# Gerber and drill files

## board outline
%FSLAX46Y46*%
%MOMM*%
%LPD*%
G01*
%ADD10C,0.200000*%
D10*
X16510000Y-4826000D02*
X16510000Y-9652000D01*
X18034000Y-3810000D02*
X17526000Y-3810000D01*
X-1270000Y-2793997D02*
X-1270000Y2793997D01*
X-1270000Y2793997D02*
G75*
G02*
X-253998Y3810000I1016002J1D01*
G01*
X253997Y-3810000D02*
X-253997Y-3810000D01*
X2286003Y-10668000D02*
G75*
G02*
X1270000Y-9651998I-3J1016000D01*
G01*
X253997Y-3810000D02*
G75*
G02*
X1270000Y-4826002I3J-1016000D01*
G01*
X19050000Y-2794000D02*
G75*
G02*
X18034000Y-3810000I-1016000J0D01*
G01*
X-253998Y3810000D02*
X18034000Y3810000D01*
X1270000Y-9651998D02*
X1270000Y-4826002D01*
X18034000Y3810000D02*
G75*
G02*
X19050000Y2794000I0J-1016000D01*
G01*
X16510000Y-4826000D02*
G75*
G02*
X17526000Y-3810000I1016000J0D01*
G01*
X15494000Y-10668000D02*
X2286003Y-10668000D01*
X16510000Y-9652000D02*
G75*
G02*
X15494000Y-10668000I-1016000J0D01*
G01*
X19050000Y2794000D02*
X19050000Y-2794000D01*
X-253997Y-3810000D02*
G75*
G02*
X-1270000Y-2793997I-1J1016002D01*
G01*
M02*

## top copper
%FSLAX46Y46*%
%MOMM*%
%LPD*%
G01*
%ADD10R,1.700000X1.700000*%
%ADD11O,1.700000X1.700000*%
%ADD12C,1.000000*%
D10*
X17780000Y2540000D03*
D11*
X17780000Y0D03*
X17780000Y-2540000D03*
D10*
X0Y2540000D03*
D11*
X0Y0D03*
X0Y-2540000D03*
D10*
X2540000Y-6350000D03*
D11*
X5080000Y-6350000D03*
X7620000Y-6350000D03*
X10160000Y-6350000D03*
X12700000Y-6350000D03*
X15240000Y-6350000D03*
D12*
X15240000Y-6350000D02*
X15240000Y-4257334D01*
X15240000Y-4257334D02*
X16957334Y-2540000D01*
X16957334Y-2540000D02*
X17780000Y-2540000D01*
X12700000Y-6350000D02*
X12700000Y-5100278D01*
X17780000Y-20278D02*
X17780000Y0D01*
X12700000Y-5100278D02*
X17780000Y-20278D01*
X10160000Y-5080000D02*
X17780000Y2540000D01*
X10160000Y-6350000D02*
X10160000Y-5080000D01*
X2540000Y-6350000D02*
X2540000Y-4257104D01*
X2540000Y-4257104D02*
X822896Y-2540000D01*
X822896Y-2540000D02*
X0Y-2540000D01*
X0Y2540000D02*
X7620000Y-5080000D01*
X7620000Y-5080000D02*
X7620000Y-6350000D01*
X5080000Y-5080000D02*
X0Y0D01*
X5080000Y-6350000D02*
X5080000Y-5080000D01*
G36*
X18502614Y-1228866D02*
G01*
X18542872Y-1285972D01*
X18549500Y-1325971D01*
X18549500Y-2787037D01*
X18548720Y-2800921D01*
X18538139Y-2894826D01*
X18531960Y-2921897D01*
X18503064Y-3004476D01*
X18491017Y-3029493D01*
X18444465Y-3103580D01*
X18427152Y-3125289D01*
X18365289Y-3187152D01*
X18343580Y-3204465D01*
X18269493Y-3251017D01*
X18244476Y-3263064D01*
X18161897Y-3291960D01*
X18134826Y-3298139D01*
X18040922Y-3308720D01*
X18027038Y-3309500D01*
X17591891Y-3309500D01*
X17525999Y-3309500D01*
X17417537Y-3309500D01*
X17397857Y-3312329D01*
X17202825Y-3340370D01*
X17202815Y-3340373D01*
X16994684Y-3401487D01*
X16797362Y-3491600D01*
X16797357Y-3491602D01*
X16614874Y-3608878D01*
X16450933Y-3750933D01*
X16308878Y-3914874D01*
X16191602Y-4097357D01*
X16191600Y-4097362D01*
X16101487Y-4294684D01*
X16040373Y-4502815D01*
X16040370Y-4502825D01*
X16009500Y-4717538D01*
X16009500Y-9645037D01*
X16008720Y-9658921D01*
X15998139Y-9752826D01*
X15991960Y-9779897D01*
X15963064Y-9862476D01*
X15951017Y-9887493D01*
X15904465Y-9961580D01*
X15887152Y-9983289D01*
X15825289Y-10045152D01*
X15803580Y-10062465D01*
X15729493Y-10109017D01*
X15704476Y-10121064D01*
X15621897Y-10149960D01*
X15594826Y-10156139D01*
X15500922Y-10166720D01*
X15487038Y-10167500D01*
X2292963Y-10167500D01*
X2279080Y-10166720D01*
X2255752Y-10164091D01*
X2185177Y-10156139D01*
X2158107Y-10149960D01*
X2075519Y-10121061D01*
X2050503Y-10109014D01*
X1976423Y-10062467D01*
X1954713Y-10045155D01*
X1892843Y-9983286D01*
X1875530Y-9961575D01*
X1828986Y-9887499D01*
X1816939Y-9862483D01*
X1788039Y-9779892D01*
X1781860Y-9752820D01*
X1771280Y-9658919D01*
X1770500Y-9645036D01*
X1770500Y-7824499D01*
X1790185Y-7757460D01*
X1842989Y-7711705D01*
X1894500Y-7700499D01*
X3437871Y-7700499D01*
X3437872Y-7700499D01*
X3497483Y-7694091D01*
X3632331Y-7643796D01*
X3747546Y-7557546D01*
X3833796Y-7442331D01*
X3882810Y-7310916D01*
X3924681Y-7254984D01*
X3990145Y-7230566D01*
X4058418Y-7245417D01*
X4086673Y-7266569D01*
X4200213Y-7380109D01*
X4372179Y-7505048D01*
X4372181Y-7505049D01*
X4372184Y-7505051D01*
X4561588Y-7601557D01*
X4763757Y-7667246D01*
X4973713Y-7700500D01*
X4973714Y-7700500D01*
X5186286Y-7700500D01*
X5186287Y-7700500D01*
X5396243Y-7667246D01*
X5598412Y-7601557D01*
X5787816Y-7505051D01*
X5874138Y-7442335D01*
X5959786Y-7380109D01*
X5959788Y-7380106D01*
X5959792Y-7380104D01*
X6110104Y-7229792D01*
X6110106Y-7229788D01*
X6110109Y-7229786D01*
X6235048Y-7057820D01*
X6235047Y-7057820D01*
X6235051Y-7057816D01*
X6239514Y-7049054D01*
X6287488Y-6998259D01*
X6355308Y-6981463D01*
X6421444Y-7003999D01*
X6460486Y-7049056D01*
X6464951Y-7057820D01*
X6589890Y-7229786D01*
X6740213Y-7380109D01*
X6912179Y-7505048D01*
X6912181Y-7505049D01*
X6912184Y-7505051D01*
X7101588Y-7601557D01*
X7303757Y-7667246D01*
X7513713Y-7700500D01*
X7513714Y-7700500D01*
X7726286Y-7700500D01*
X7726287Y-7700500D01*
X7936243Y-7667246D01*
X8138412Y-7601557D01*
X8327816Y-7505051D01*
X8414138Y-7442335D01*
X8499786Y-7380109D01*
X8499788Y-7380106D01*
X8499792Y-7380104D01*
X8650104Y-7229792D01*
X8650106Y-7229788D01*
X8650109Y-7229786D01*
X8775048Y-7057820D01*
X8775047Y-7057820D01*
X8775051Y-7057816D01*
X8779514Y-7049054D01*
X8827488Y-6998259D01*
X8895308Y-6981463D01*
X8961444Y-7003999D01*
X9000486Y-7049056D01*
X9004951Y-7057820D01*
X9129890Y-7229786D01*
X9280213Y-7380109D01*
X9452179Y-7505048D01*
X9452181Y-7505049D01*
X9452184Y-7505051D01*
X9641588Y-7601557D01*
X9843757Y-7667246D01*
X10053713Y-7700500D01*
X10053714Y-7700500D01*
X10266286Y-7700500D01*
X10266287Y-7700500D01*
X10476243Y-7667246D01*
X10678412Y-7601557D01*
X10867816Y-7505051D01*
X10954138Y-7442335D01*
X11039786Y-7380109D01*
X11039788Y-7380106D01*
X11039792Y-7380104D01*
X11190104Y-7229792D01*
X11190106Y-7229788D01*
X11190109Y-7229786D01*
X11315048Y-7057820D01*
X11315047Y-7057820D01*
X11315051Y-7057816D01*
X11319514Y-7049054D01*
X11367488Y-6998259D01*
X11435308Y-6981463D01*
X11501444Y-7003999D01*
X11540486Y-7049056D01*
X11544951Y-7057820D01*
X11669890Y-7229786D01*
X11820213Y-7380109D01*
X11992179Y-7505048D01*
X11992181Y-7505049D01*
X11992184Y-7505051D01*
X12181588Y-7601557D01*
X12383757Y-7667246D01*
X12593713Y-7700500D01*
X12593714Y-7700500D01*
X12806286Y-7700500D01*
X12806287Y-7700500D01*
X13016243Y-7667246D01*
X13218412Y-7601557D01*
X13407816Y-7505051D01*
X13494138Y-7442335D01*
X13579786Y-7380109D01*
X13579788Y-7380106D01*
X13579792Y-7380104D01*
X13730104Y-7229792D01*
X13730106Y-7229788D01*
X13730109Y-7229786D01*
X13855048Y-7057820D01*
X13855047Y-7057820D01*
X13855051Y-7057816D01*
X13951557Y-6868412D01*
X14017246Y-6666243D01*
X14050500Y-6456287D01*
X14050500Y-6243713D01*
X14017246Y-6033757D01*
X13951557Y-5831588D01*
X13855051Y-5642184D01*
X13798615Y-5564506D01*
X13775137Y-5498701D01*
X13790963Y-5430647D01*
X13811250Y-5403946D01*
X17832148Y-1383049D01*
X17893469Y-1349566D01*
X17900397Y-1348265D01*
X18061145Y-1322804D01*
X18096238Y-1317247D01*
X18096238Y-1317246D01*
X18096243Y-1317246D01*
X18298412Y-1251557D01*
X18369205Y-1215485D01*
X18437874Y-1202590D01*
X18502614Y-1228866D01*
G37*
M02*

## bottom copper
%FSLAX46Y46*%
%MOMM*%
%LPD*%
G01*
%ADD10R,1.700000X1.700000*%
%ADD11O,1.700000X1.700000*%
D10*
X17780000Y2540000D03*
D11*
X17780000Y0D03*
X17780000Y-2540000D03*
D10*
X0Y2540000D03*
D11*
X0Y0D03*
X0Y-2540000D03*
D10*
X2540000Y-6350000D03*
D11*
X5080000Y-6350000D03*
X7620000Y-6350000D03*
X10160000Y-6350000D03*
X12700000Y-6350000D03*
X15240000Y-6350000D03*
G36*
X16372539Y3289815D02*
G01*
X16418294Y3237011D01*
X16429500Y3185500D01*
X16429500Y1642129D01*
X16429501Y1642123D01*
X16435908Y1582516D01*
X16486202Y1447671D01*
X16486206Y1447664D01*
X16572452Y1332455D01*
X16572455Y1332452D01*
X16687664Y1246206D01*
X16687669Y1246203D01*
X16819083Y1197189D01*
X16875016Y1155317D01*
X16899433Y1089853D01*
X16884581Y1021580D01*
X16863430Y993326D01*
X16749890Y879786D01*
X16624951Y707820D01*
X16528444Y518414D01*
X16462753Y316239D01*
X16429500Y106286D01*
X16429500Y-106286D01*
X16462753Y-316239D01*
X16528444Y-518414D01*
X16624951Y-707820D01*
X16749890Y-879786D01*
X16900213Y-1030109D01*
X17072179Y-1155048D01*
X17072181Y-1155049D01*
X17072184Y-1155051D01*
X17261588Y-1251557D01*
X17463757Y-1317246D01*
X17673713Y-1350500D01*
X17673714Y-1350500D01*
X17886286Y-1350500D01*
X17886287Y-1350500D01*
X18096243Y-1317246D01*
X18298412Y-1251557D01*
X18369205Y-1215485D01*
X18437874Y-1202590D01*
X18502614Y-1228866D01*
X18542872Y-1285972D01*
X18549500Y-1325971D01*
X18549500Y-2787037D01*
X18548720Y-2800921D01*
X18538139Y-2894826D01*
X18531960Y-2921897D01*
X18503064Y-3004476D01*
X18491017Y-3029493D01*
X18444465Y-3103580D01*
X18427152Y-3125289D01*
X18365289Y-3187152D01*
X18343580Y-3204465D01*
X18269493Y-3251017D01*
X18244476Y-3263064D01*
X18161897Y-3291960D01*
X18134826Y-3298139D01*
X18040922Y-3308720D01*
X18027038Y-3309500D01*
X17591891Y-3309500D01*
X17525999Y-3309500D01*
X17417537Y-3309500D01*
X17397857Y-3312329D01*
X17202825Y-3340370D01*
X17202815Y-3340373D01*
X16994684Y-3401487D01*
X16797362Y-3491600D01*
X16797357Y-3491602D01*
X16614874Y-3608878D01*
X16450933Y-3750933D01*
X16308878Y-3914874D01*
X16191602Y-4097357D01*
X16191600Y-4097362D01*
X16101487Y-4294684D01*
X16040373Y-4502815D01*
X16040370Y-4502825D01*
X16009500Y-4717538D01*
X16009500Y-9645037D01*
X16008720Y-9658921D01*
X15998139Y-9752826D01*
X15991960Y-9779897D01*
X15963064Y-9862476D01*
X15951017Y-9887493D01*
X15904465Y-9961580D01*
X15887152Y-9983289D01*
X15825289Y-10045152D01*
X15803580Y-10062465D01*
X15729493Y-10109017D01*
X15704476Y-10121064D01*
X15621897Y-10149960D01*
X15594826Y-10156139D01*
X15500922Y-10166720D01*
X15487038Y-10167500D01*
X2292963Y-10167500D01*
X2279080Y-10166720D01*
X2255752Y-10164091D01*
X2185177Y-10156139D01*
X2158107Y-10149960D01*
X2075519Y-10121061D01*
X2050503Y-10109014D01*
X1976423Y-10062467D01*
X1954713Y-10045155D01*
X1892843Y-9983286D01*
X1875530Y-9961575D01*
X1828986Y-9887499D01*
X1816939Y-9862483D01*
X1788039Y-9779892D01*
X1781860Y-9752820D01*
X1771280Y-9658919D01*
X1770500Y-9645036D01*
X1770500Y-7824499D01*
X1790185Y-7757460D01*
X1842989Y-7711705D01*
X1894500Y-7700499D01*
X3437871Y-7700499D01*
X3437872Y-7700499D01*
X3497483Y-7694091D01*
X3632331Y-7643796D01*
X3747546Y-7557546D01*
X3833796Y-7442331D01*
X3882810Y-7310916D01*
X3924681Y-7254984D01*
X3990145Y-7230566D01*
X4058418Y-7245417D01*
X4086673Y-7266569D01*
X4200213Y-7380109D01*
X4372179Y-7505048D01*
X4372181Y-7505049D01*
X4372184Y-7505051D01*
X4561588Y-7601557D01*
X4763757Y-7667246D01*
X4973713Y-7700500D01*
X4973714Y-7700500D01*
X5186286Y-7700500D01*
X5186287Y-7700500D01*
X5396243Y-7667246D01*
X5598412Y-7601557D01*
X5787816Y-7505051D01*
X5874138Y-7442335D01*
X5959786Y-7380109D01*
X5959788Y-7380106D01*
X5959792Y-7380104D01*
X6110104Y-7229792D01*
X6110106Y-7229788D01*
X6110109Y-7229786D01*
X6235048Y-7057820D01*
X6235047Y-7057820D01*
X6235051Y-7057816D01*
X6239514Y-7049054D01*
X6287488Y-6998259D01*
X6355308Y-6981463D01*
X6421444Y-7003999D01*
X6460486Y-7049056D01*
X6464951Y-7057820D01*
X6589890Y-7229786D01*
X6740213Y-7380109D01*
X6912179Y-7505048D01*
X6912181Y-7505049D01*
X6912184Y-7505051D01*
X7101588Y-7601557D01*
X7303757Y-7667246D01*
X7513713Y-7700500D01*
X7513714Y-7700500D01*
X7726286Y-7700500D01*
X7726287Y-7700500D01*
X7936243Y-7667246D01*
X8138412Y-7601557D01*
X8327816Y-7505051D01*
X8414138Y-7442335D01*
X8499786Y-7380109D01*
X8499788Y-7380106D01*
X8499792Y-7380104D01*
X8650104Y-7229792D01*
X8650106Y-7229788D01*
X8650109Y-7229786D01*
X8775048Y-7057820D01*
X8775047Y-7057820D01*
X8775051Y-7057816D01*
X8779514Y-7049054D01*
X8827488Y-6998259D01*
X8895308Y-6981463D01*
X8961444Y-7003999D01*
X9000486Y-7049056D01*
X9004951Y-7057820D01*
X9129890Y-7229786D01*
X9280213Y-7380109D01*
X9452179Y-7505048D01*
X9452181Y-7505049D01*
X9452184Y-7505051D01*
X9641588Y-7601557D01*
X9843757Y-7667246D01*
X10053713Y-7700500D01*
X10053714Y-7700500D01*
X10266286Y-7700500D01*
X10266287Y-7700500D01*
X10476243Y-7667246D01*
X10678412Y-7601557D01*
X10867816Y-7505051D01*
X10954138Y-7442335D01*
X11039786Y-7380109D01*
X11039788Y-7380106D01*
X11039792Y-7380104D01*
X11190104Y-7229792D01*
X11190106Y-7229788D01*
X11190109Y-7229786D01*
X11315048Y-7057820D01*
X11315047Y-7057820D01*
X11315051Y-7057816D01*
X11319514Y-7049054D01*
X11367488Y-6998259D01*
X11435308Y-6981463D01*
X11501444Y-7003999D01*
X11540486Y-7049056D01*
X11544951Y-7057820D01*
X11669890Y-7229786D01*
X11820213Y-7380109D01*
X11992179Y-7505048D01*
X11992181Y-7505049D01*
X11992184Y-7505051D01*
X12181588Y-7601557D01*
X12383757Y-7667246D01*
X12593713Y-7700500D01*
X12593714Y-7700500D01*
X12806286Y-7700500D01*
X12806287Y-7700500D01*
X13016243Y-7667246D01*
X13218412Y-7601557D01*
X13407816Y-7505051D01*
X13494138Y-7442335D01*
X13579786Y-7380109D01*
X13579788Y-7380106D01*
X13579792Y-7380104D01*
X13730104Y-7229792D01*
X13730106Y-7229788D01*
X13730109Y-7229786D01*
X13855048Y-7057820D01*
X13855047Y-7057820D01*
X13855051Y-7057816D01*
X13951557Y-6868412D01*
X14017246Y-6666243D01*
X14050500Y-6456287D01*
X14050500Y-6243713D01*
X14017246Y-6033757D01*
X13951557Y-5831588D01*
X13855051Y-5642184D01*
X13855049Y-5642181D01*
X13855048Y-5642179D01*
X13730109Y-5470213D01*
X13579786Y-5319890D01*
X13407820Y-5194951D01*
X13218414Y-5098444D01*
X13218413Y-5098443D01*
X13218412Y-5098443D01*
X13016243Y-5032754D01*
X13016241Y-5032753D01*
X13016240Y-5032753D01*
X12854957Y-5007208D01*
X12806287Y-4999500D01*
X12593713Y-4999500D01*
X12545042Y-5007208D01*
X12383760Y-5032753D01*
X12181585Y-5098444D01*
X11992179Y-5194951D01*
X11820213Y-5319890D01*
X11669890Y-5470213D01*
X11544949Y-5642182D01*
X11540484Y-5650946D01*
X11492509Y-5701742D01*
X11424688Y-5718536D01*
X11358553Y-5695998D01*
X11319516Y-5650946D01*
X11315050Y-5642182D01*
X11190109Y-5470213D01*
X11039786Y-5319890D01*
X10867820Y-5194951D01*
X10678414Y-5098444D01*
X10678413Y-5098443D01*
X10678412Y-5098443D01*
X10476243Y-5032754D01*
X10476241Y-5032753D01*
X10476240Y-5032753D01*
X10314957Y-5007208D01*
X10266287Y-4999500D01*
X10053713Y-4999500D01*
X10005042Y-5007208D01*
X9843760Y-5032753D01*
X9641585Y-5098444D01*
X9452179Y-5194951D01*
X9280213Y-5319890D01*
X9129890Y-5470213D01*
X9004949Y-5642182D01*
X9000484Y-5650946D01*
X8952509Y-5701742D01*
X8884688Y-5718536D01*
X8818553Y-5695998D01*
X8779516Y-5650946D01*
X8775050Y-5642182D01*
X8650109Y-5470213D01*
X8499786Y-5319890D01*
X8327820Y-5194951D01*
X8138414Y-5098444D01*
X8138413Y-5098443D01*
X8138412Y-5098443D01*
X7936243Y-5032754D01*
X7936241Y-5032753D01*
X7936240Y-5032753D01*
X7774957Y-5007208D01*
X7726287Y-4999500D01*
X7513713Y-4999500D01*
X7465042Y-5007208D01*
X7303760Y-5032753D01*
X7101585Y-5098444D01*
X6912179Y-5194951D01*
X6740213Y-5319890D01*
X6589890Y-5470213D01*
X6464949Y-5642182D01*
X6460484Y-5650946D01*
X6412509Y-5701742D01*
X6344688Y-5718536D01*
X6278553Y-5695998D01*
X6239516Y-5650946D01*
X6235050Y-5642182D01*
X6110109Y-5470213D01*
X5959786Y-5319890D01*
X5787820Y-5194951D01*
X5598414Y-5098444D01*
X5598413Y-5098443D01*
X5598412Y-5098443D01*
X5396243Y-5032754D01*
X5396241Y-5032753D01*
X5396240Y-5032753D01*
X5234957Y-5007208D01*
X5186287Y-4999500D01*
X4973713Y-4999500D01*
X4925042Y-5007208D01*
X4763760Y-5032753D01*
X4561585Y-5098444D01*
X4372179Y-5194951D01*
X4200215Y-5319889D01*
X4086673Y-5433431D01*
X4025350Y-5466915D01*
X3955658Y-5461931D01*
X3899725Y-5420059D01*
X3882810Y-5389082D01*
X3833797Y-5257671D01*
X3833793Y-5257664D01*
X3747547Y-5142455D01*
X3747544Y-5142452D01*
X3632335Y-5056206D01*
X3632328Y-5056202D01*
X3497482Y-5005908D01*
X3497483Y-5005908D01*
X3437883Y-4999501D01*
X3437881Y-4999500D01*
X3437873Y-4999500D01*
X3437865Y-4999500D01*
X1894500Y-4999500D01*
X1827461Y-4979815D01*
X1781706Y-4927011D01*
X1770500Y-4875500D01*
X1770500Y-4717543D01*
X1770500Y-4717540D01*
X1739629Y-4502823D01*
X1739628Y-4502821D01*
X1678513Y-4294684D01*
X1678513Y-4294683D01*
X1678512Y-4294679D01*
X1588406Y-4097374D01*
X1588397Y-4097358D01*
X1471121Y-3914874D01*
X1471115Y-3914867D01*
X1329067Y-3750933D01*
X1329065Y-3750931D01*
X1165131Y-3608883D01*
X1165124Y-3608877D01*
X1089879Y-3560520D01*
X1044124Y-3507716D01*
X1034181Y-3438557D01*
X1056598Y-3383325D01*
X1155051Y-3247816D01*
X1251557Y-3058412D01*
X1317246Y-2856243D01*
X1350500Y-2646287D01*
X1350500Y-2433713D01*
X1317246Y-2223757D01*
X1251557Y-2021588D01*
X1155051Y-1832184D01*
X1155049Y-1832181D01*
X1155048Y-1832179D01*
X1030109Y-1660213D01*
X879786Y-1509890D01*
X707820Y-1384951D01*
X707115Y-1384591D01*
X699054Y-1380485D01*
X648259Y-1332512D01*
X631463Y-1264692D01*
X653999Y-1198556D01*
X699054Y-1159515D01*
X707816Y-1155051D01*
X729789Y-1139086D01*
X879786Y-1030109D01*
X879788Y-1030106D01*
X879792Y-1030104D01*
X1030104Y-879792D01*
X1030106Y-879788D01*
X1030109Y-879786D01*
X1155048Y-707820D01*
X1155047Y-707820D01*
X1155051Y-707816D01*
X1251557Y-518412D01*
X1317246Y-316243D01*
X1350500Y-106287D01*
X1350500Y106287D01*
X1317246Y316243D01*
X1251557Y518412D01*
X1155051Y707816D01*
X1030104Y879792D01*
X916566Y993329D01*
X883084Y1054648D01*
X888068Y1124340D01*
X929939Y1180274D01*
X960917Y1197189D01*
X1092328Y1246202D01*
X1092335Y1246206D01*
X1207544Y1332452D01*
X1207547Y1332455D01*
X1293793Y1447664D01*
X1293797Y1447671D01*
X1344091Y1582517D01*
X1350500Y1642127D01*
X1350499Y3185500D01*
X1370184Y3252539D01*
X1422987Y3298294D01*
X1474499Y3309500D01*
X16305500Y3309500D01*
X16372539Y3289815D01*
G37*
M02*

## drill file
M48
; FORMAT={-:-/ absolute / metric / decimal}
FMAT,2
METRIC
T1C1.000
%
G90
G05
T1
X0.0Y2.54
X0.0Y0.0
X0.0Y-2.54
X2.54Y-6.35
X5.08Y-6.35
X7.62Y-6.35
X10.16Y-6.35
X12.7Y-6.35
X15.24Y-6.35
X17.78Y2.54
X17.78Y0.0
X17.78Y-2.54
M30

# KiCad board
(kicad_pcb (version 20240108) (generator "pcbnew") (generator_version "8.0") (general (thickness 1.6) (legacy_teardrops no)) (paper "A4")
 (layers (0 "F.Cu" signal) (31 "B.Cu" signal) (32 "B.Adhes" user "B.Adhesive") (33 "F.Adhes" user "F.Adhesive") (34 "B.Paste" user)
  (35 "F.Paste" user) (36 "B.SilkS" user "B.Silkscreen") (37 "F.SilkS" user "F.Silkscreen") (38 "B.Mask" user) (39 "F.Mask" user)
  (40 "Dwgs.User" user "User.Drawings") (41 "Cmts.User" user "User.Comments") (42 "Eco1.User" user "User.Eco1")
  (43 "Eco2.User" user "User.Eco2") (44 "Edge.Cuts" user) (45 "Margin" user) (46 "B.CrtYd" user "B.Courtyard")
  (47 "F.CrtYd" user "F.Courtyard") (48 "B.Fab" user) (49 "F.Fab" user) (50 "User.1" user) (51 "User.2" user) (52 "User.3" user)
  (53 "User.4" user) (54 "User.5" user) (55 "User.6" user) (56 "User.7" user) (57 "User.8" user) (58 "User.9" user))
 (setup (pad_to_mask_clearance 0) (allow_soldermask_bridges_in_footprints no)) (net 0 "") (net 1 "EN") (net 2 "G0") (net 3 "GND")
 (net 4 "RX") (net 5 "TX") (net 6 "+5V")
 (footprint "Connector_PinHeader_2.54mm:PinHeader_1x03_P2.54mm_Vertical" (layer "F.Cu") (at 17.78 -2.54)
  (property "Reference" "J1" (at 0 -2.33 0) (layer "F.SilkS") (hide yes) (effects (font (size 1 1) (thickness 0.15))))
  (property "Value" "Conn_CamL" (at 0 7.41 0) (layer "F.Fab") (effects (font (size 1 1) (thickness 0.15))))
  (pad "1" thru_hole rect (at 0 0) (size 1.7 1.7) (drill 1) (layers "*.Cu" "*.Mask") (remove_unused_layers no) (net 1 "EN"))
  (pad "2" thru_hole oval (at 0 2.54) (size 1.7 1.7) (drill 1) (layers "*.Cu" "*.Mask") (remove_unused_layers no) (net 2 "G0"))
  (pad "3" thru_hole oval (at 0 5.08) (size 1.7 1.7) (drill 1) (layers "*.Cu" "*.Mask") (remove_unused_layers no) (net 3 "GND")))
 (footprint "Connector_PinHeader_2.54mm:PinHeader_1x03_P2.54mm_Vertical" (layer "F.Cu") (at 0 -2.54)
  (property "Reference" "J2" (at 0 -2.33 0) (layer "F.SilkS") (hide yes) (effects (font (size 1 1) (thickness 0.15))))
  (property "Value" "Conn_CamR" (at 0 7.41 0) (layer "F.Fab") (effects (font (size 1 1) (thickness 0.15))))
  (pad "1" thru_hole rect (at 0 0) (size 1.7 1.7) (drill 1) (layers "*.Cu" "*.Mask") (remove_unused_layers no) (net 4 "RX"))
  (pad "2" thru_hole oval (at 0 2.54) (size 1.7 1.7) (drill 1) (layers "*.Cu" "*.Mask") (remove_unused_layers no) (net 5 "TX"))
  (pad "3" thru_hole oval (at 0 5.08) (size 1.7 1.7) (drill 1) (layers "*.Cu" "*.Mask") (remove_unused_layers no) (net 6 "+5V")))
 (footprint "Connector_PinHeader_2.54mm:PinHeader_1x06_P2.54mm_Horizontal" (layer "B.Cu") (at 2.54 6.35 -90)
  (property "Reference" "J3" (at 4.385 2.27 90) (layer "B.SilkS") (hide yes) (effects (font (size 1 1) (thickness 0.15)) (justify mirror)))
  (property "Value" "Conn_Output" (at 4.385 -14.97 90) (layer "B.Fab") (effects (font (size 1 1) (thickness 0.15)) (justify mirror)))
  (pad "1" thru_hole rect (at 0 0 270) (size 1.7 1.7) (drill 1) (layers "*.Cu" "*.Mask") (remove_unused_layers no) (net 6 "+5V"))
  (pad "2" thru_hole oval (at 0 -2.54 270) (size 1.7 1.7) (drill 1) (layers "*.Cu" "*.Mask") (remove_unused_layers no) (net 5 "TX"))
  (pad "3" thru_hole oval (at 0 -5.08 270) (size 1.7 1.7) (drill 1) (layers "*.Cu" "*.Mask") (remove_unused_layers no) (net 4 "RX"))
  (pad "4" thru_hole oval (at 0 -7.62 270) (size 1.7 1.7) (drill 1) (layers "*.Cu" "*.Mask") (remove_unused_layers no) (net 1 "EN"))
  (pad "5" thru_hole oval (at 0 -10.16 270) (size 1.7 1.7) (drill 1) (layers "*.Cu" "*.Mask") (remove_unused_layers no) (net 2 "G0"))
  (pad "6" thru_hole oval (at 0 -12.7 270) (size 1.7 1.7) (drill 1) (layers "*.Cu" "*.Mask") (remove_unused_layers no) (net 3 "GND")))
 (gr_line (start 16.51 4.826) (end 16.51 9.652) (stroke (width 0.2) (type default)) (layer "Edge.Cuts"))
 (gr_line (start 18.034 3.81) (end 17.526 3.81) (stroke (width 0.2) (type default)) (layer "Edge.Cuts"))
 (gr_line (start -1.27 2.793997) (end -1.27 -2.793997) (stroke (width 0.2) (type default)) (layer "Edge.Cuts"))
 (gr_arc (start -1.27 -2.793997) (mid -0.97242 -3.51242) (end -0.253998 -3.81) (stroke (width 0.2) (type default)) (layer "Edge.Cuts"))
 (gr_line (start 0.253997 3.81) (end -0.253997 3.81) (stroke (width 0.2) (type default)) (layer "Edge.Cuts"))
 (gr_arc (start 2.286003 10.668) (mid 1.56758 10.37042) (end 1.27 9.651998) (stroke (width 0.2) (type default)) (layer "Edge.Cuts"))
 (gr_arc (start 0.253997 3.81) (mid 0.97242 4.10758) (end 1.27 4.826002) (stroke (width 0.2) (type default)) (layer "Edge.Cuts"))
 (gr_arc (start 19.05 2.794) (mid 18.75242 3.51242) (end 18.034 3.81) (stroke (width 0.2) (type default)) (layer "Edge.Cuts"))
 (gr_line (start -0.253998 -3.81) (end 18.034 -3.81) (stroke (width 0.2) (type default)) (layer "Edge.Cuts"))
 (gr_line (start 1.27 9.651998) (end 1.27 4.826002) (stroke (width 0.2) (type default)) (layer "Edge.Cuts"))
 (gr_arc (start 18.034 -3.81) (mid 18.75242 -3.51242) (end 19.05 -2.794) (stroke (width 0.2) (type default)) (layer "Edge.Cuts"))
 (gr_arc (start 16.51 4.826) (mid 16.80758 4.10758) (end 17.526 3.81) (stroke (width 0.2) (type default)) (layer "Edge.Cuts"))
 (gr_line (start 15.494 10.668) (end 2.286003 10.668) (stroke (width 0.2) (type default)) (layer "Edge.Cuts"))
 (gr_arc (start 16.51 9.652) (mid 16.21242 10.37042) (end 15.494 10.668) (stroke (width 0.2) (type default)) (layer "Edge.Cuts"))
 (gr_line (start 19.05 -2.794) (end 19.05 2.794) (stroke (width 0.2) (type default)) (layer "Edge.Cuts"))
 (gr_arc (start -0.253997 3.81) (mid -0.97242 3.51242) (end -1.27 2.793997) (stroke (width 0.2) (type default)) (layer "Edge.Cuts"))
 (segment (start 15.24 6.35) (end 15.24 4.257334) (width 1) (layer "F.Cu") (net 3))
 (segment (start 15.24 4.257334) (end 16.957334 2.54) (width 1) (layer "F.Cu") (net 3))
 (segment (start 16.957334 2.54) (end 17.78 2.54) (width 1) (layer "F.Cu") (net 3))
 (segment (start 12.7 6.35) (end 12.7 5.100278) (width 1) (layer "F.Cu") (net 2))
 (segment (start 17.78 0.020278) (end 17.78 0) (width 1) (layer "F.Cu") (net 2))
 (segment (start 12.7 5.100278) (end 17.78 0.020278) (width 1) (layer "F.Cu") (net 2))
 (segment (start 10.16 5.08) (end 17.78 -2.54) (width 1) (layer "F.Cu") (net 1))
 (segment (start 10.16 6.35) (end 10.16 5.08) (width 1) (layer "F.Cu") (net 1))
 (segment (start 2.54 6.35) (end 2.54 4.257104) (width 1) (layer "F.Cu") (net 6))
 (segment (start 2.54 4.257104) (end 0.822896 2.54) (width 1) (layer "F.Cu") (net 6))
 (segment (start 0.822896 2.54) (end 0 2.54) (width 1) (layer "F.Cu") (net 6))
 (segment (start 0 -2.54) (end 7.62 5.08) (width 1) (layer "F.Cu") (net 4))
 (segment (start 7.62 5.08) (end 7.62 6.35) (width 1) (layer "F.Cu") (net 4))
 (segment (start 5.08 5.08) (end 0 0) (width 1) (layer "F.Cu") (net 5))
 (segment (start 5.08 6.35) (end 5.08 5.08) (width 1) (layer "F.Cu") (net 5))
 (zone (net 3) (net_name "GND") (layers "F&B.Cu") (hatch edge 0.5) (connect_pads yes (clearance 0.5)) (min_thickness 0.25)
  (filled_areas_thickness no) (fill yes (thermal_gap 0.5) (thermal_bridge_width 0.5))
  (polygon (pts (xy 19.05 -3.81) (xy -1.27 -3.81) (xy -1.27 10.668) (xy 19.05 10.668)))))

